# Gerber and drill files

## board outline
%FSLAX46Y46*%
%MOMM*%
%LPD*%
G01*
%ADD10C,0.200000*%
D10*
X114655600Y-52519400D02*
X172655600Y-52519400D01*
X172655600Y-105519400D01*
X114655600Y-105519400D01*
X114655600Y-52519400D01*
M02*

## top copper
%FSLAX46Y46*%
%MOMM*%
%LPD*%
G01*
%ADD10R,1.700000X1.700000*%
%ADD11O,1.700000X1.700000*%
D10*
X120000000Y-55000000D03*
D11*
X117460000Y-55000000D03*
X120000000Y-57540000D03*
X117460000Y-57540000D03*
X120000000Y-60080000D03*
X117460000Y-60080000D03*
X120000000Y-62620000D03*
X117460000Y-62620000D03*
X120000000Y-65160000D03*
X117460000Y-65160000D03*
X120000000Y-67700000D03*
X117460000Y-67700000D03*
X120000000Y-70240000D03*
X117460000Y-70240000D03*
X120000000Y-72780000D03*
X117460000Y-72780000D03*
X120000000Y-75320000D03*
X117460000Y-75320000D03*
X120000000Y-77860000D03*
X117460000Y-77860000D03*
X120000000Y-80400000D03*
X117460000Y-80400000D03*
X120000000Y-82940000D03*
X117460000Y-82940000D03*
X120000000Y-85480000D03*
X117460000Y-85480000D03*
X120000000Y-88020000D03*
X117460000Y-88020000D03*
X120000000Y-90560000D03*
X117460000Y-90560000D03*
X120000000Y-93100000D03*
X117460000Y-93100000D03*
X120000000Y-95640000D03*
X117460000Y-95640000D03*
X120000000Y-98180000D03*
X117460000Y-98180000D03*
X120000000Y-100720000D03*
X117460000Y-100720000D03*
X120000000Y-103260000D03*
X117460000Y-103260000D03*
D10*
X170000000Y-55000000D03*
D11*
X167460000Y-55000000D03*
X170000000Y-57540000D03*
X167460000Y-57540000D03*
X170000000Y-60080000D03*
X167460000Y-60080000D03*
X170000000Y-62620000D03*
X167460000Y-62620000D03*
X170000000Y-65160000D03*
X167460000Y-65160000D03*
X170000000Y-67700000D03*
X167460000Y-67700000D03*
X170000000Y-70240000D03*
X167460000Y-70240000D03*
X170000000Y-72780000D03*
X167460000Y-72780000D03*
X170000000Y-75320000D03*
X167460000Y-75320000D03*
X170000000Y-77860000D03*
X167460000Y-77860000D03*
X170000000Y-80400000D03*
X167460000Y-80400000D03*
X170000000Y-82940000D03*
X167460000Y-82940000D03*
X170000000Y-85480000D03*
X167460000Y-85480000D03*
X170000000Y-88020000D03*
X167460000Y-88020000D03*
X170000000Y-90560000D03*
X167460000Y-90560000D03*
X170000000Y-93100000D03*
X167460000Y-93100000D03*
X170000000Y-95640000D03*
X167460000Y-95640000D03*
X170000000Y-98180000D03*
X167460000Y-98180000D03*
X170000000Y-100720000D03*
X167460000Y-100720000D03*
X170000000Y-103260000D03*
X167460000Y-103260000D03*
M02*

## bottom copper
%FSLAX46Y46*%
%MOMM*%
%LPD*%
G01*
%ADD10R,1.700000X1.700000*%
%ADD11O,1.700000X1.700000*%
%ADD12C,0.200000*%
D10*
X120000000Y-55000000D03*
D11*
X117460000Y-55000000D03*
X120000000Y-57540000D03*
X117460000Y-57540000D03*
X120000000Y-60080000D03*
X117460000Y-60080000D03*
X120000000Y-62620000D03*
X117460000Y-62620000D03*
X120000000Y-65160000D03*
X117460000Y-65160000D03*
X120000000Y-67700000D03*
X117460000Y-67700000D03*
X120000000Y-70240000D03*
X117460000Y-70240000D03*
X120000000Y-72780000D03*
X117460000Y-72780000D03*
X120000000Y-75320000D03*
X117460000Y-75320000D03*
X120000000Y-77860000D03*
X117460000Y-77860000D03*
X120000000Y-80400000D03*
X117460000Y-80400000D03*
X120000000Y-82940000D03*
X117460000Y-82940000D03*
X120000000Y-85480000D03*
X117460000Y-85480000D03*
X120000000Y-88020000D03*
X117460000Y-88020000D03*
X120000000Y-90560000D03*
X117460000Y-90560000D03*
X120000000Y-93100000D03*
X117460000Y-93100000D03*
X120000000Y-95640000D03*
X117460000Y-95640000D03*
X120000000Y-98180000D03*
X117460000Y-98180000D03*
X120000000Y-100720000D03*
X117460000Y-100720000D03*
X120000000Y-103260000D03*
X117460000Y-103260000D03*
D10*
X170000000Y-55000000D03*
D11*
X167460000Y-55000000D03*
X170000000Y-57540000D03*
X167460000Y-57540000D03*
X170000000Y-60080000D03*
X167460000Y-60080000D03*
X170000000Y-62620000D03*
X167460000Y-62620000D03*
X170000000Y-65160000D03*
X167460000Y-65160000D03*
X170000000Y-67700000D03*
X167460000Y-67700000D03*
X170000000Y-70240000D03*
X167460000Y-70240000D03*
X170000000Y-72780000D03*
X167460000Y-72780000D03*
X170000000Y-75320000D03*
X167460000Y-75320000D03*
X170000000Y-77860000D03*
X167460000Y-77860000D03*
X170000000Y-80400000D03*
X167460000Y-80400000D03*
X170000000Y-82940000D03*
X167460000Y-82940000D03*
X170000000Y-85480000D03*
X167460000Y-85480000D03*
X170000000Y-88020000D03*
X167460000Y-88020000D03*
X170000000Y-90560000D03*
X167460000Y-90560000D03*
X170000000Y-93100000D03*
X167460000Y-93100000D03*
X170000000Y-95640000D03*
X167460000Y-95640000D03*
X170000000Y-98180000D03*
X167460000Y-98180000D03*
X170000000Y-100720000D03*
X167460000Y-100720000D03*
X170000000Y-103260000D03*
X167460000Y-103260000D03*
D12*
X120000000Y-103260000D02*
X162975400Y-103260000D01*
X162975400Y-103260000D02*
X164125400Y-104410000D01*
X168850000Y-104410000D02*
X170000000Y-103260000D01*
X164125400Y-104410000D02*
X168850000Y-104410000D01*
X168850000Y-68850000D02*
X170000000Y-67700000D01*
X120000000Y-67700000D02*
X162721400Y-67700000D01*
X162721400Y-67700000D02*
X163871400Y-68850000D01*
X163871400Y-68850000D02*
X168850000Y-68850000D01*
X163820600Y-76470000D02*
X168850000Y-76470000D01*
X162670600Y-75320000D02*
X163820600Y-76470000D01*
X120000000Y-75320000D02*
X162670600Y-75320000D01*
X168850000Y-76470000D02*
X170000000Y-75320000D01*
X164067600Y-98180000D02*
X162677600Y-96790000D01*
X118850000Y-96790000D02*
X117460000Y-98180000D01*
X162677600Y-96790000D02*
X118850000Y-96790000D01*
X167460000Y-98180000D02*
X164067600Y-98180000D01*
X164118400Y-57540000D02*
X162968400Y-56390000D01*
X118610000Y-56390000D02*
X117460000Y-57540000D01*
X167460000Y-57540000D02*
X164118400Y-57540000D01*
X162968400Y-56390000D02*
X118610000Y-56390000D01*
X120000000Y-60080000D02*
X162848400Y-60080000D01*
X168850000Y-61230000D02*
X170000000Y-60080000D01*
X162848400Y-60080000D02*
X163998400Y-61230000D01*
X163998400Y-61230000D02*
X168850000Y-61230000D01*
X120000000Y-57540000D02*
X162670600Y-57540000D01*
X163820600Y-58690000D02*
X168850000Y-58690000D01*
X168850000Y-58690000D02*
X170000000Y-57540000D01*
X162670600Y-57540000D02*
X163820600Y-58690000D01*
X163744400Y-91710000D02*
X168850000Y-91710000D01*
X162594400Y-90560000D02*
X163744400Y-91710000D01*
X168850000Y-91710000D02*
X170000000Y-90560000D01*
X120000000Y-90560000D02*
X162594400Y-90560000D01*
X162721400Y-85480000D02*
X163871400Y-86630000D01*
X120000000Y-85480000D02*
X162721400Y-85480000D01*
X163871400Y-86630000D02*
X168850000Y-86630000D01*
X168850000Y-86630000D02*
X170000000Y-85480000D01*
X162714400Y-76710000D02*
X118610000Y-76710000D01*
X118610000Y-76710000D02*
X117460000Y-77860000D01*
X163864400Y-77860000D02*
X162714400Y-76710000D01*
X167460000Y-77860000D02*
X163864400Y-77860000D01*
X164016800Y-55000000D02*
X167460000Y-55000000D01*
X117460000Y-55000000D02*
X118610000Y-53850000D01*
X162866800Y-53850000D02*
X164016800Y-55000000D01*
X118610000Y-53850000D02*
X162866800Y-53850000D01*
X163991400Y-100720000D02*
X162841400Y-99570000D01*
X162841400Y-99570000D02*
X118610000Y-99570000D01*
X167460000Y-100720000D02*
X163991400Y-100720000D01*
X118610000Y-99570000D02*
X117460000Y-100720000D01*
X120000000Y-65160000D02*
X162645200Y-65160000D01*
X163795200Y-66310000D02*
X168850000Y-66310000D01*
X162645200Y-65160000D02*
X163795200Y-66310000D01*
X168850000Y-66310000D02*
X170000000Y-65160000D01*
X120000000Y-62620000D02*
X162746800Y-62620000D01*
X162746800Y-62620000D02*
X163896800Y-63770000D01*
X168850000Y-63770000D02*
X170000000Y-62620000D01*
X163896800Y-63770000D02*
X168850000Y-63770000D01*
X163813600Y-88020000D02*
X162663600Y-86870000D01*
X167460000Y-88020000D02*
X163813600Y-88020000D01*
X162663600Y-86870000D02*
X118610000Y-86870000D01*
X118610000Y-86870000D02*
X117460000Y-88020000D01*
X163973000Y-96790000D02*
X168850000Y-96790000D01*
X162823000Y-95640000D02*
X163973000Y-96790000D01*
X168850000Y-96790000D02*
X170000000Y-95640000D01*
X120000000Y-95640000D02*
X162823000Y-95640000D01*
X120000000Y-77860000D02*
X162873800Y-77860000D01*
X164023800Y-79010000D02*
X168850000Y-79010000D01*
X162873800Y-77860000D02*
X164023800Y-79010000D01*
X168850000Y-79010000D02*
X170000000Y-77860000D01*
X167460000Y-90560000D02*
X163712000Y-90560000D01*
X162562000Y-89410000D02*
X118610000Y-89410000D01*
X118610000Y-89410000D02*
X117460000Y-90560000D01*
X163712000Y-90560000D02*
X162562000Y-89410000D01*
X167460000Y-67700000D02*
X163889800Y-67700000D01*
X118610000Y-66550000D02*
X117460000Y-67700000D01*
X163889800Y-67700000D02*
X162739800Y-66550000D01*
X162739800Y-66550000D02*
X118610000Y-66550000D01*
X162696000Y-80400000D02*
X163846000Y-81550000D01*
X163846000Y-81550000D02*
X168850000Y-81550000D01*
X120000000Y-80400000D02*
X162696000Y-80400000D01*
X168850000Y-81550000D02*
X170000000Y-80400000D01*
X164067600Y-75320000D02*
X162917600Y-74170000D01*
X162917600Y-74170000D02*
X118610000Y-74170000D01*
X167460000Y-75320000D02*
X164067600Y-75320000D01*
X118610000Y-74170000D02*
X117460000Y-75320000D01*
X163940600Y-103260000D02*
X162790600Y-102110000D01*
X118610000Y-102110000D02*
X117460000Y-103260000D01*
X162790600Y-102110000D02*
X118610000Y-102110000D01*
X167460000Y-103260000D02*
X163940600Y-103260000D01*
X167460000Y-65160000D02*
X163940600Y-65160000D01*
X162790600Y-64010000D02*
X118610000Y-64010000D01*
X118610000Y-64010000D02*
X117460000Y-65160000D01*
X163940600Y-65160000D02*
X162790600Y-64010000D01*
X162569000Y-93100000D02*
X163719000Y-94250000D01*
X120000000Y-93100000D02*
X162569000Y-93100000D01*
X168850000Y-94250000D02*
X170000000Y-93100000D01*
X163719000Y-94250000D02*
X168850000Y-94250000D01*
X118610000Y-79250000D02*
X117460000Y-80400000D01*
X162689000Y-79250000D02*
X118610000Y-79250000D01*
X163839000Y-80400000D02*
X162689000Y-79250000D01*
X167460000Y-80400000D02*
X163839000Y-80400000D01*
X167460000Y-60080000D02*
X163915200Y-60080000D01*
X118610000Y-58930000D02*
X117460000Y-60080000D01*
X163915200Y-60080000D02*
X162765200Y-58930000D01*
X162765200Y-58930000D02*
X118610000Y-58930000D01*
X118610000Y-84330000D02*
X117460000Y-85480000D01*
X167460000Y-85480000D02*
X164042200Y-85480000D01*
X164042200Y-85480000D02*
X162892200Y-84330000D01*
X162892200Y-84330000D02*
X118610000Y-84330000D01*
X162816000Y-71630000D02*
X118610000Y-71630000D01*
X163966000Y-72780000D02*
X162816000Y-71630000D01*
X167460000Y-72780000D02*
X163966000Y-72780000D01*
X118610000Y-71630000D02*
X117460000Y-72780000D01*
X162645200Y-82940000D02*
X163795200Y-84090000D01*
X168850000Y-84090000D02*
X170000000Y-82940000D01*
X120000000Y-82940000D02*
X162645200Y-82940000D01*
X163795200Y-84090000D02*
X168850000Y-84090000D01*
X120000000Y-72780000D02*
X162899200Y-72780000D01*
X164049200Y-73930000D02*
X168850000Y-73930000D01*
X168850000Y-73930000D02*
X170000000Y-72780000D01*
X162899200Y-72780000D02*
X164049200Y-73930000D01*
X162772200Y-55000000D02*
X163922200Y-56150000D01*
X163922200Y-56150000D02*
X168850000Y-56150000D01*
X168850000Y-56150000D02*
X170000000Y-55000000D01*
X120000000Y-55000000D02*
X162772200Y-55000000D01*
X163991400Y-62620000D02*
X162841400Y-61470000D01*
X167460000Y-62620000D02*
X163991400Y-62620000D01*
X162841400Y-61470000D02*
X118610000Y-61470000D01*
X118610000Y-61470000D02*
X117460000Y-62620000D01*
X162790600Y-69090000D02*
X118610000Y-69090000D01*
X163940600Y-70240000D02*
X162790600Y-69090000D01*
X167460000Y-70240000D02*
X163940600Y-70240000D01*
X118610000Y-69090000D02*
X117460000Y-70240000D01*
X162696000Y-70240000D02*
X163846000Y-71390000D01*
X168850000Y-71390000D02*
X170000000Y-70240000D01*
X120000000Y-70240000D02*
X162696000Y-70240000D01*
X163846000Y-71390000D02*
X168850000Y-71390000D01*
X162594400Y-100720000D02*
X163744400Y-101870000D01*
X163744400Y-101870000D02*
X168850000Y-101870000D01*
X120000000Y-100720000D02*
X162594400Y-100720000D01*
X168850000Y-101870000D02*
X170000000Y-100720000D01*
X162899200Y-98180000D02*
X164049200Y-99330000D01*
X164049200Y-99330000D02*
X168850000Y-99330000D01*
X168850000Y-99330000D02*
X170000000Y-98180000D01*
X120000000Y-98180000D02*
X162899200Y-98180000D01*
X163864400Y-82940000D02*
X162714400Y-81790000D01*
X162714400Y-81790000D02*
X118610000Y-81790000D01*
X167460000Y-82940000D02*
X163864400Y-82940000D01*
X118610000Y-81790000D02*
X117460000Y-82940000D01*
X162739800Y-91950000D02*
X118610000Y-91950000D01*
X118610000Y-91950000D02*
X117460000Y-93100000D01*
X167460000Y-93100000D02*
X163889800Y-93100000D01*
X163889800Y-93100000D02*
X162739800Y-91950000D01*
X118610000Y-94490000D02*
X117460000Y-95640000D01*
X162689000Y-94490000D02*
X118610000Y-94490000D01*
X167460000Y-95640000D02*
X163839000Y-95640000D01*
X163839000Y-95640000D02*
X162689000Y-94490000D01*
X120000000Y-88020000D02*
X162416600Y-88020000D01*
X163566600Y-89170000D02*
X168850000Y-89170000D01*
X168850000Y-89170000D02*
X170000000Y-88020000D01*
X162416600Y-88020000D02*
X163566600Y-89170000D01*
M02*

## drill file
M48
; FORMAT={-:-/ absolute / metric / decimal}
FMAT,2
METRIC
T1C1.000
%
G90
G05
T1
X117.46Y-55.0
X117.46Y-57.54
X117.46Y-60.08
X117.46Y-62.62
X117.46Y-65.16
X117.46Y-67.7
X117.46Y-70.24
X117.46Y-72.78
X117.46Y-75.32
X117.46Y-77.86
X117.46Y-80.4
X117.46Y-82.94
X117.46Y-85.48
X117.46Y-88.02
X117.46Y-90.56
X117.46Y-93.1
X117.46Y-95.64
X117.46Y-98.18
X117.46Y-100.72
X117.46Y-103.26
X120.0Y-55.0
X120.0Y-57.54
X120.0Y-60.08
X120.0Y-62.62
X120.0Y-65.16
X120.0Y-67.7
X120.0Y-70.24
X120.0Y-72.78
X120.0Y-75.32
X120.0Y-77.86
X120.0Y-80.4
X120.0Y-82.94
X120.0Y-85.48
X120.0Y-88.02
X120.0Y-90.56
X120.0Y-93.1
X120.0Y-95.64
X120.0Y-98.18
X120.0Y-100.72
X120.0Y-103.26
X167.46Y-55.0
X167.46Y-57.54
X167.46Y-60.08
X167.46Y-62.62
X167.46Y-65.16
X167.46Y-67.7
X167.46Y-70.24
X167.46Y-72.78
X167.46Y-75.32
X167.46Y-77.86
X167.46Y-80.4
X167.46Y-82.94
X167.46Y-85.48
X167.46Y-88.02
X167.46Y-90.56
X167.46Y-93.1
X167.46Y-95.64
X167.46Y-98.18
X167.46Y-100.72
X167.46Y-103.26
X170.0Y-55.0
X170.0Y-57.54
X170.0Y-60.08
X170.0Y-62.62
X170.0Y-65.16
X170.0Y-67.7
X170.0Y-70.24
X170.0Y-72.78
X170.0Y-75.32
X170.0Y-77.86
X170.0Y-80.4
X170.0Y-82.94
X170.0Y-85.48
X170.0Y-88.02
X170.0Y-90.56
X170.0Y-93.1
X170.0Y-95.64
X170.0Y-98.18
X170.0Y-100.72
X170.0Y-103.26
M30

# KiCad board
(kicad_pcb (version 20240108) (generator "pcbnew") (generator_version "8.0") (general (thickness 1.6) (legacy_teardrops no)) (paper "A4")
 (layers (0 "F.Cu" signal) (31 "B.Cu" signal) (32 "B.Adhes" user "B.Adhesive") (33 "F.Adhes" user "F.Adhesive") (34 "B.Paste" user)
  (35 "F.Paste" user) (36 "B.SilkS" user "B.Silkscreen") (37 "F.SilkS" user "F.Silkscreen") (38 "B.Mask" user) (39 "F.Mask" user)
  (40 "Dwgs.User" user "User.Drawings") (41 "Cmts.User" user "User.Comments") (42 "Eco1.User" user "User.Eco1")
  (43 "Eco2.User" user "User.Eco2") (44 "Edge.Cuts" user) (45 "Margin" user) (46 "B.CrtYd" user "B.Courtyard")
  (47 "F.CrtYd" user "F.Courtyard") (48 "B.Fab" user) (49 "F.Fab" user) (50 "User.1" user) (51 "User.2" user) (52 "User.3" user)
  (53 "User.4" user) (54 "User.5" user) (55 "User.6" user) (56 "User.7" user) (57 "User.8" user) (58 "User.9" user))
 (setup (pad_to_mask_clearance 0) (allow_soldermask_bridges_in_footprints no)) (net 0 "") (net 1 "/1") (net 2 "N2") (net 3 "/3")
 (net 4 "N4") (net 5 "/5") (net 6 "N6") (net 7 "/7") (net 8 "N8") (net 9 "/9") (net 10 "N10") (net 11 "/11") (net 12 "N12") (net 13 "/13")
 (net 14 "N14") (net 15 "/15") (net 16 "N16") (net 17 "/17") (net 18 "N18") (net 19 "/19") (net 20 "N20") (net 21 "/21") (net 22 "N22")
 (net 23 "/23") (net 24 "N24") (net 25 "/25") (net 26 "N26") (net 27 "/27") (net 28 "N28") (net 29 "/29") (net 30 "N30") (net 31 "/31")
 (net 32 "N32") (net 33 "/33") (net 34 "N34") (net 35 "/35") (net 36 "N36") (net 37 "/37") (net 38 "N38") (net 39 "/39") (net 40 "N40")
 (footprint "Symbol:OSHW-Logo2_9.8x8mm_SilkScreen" (layer "F.Cu") (at 160.274 97.8408 90)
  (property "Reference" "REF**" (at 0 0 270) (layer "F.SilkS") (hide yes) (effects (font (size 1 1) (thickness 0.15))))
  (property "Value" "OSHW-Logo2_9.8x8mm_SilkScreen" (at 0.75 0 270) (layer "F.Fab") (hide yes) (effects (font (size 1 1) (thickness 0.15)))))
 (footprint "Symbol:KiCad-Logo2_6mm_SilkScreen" (layer "F.Cu") (at 159.512 62.7634 90)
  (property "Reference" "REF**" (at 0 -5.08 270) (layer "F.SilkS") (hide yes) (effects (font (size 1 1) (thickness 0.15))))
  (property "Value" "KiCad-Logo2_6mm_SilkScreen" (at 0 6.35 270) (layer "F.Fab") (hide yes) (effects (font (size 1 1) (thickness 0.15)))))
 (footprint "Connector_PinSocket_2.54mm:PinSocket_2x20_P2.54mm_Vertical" (layer "F.Cu") (at 120 55)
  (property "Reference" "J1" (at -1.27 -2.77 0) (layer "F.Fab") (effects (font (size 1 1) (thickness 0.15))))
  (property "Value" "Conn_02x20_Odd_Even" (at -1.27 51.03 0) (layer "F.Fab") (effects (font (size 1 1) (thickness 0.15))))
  (pad "1" thru_hole rect (at 0 0) (size 1.7 1.7) (drill 1) (layers "*.Cu" "*.Mask") (remove_unused_layers no) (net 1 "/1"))
  (pad "2" thru_hole oval (at -2.54 0) (size 1.7 1.7) (drill 1) (layers "*.Cu" "*.Mask") (remove_unused_layers no) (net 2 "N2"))
  (pad "3" thru_hole oval (at 0 2.54) (size 1.7 1.7) (drill 1) (layers "*.Cu" "*.Mask") (remove_unused_layers no) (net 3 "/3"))
  (pad "4" thru_hole oval (at -2.54 2.54) (size 1.7 1.7) (drill 1) (layers "*.Cu" "*.Mask") (remove_unused_layers no) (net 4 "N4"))
  (pad "5" thru_hole oval (at 0 5.08) (size 1.7 1.7) (drill 1) (layers "*.Cu" "*.Mask") (remove_unused_layers no) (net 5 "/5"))
  (pad "6" thru_hole oval (at -2.54 5.08) (size 1.7 1.7) (drill 1) (layers "*.Cu" "*.Mask") (remove_unused_layers no) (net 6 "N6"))
  (pad "7" thru_hole oval (at 0 7.62) (size 1.7 1.7) (drill 1) (layers "*.Cu" "*.Mask") (remove_unused_layers no) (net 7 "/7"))
  (pad "8" thru_hole oval (at -2.54 7.62) (size 1.7 1.7) (drill 1) (layers "*.Cu" "*.Mask") (remove_unused_layers no) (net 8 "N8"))
  (pad "9" thru_hole oval (at 0 10.16) (size 1.7 1.7) (drill 1) (layers "*.Cu" "*.Mask") (remove_unused_layers no) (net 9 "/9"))
  (pad "10" thru_hole oval (at -2.54 10.16) (size 1.7 1.7) (drill 1) (layers "*.Cu" "*.Mask") (remove_unused_layers no) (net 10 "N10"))
  (pad "11" thru_hole oval (at 0 12.7) (size 1.7 1.7) (drill 1) (layers "*.Cu" "*.Mask") (remove_unused_layers no) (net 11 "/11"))
  (pad "12" thru_hole oval (at -2.54 12.7) (size 1.7 1.7) (drill 1) (layers "*.Cu" "*.Mask") (remove_unused_layers no) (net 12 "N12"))
  (pad "13" thru_hole oval (at 0 15.24) (size 1.7 1.7) (drill 1) (layers "*.Cu" "*.Mask") (remove_unused_layers no) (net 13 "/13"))
  (pad "14" thru_hole oval (at -2.54 15.24) (size 1.7 1.7) (drill 1) (layers "*.Cu" "*.Mask") (remove_unused_layers no) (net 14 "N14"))
  (pad "15" thru_hole oval (at 0 17.78) (size 1.7 1.7) (drill 1) (layers "*.Cu" "*.Mask") (remove_unused_layers no) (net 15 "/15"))
  (pad "16" thru_hole oval (at -2.54 17.78) (size 1.7 1.7) (drill 1) (layers "*.Cu" "*.Mask") (remove_unused_layers no) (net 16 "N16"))
  (pad "17" thru_hole oval (at 0 20.32) (size 1.7 1.7) (drill 1) (layers "*.Cu" "*.Mask") (remove_unused_layers no) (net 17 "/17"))
  (pad "18" thru_hole oval (at -2.54 20.32) (size 1.7 1.7) (drill 1) (layers "*.Cu" "*.Mask") (remove_unused_layers no) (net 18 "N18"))
  (pad "19" thru_hole oval (at 0 22.86) (size 1.7 1.7) (drill 1) (layers "*.Cu" "*.Mask") (remove_unused_layers no) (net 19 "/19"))
  (pad "20" thru_hole oval (at -2.54 22.86) (size 1.7 1.7) (drill 1) (layers "*.Cu" "*.Mask") (remove_unused_layers no) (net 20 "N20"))
  (pad "21" thru_hole oval (at 0 25.4) (size 1.7 1.7) (drill 1) (layers "*.Cu" "*.Mask") (remove_unused_layers no) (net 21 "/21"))
  (pad "22" thru_hole oval (at -2.54 25.4) (size 1.7 1.7) (drill 1) (layers "*.Cu" "*.Mask") (remove_unused_layers no) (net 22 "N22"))
  (pad "23" thru_hole oval (at 0 27.94) (size 1.7 1.7) (drill 1) (layers "*.Cu" "*.Mask") (remove_unused_layers no) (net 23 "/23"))
  (pad "24" thru_hole oval (at -2.54 27.94) (size 1.7 1.7) (drill 1) (layers "*.Cu" "*.Mask") (remove_unused_layers no) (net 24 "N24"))
  (pad "25" thru_hole oval (at 0 30.48) (size 1.7 1.7) (drill 1) (layers "*.Cu" "*.Mask") (remove_unused_layers no) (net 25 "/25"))
  (pad "26" thru_hole oval (at -2.54 30.48) (size 1.7 1.7) (drill 1) (layers "*.Cu" "*.Mask") (remove_unused_layers no) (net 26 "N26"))
  (pad "27" thru_hole oval (at 0 33.02) (size 1.7 1.7) (drill 1) (layers "*.Cu" "*.Mask") (remove_unused_layers no) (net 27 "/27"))
  (pad "28" thru_hole oval (at -2.54 33.02) (size 1.7 1.7) (drill 1) (layers "*.Cu" "*.Mask") (remove_unused_layers no) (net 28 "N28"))
  (pad "29" thru_hole oval (at 0 35.56) (size 1.7 1.7) (drill 1) (layers "*.Cu" "*.Mask") (remove_unused_layers no) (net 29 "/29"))
  (pad "30" thru_hole oval (at -2.54 35.56) (size 1.7 1.7) (drill 1) (layers "*.Cu" "*.Mask") (remove_unused_layers no) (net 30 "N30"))
  (pad "31" thru_hole oval (at 0 38.1) (size 1.7 1.7) (drill 1) (layers "*.Cu" "*.Mask") (remove_unused_layers no) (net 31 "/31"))
  (pad "32" thru_hole oval (at -2.54 38.1) (size 1.7 1.7) (drill 1) (layers "*.Cu" "*.Mask") (remove_unused_layers no) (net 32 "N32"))
  (pad "33" thru_hole oval (at 0 40.64) (size 1.7 1.7) (drill 1) (layers "*.Cu" "*.Mask") (remove_unused_layers no) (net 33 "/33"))
  (pad "34" thru_hole oval (at -2.54 40.64) (size 1.7 1.7) (drill 1) (layers "*.Cu" "*.Mask") (remove_unused_layers no) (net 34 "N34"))
  (pad "35" thru_hole oval (at 0 43.18) (size 1.7 1.7) (drill 1) (layers "*.Cu" "*.Mask") (remove_unused_layers no) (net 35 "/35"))
  (pad "36" thru_hole oval (at -2.54 43.18) (size 1.7 1.7) (drill 1) (layers "*.Cu" "*.Mask") (remove_unused_layers no) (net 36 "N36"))
  (pad "37" thru_hole oval (at 0 45.72) (size 1.7 1.7) (drill 1) (layers "*.Cu" "*.Mask") (remove_unused_layers no) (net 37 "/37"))
  (pad "38" thru_hole oval (at -2.54 45.72) (size 1.7 1.7) (drill 1) (layers "*.Cu" "*.Mask") (remove_unused_layers no) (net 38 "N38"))
  (pad "39" thru_hole oval (at 0 48.26) (size 1.7 1.7) (drill 1) (layers "*.Cu" "*.Mask") (remove_unused_layers no) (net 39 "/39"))
  (pad "40" thru_hole oval (at -2.54 48.26) (size 1.7 1.7) (drill 1) (layers "*.Cu" "*.Mask") (remove_unused_layers no) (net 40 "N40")))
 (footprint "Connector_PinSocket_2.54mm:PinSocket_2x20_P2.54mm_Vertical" (layer "F.Cu") (at 170 55)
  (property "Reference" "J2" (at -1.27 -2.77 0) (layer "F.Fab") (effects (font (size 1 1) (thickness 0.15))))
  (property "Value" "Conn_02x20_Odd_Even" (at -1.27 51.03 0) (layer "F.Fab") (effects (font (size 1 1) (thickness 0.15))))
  (pad "1" thru_hole rect (at 0 0) (size 1.7 1.7) (drill 1) (layers "*.Cu" "*.Mask") (remove_unused_layers no) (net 1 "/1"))
  (pad "2" thru_hole oval (at -2.54 0) (size 1.7 1.7) (drill 1) (layers "*.Cu" "*.Mask") (remove_unused_layers no) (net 2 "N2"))
  (pad "3" thru_hole oval (at 0 2.54) (size 1.7 1.7) (drill 1) (layers "*.Cu" "*.Mask") (remove_unused_layers no) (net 3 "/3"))
  (pad "4" thru_hole oval (at -2.54 2.54) (size 1.7 1.7) (drill 1) (layers "*.Cu" "*.Mask") (remove_unused_layers no) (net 4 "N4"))
  (pad "5" thru_hole oval (at 0 5.08) (size 1.7 1.7) (drill 1) (layers "*.Cu" "*.Mask") (remove_unused_layers no) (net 5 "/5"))
  (pad "6" thru_hole oval (at -2.54 5.08) (size 1.7 1.7) (drill 1) (layers "*.Cu" "*.Mask") (remove_unused_layers no) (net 6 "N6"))
  (pad "7" thru_hole oval (at 0 7.62) (size 1.7 1.7) (drill 1) (layers "*.Cu" "*.Mask") (remove_unused_layers no) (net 7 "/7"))
  (pad "8" thru_hole oval (at -2.54 7.62) (size 1.7 1.7) (drill 1) (layers "*.Cu" "*.Mask") (remove_unused_layers no) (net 8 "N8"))
  (pad "9" thru_hole oval (at 0 10.16) (size 1.7 1.7) (drill 1) (layers "*.Cu" "*.Mask") (remove_unused_layers no) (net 9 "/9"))
  (pad "10" thru_hole oval (at -2.54 10.16) (size 1.7 1.7) (drill 1) (layers "*.Cu" "*.Mask") (remove_unused_layers no) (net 10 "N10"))
  (pad "11" thru_hole oval (at 0 12.7) (size 1.7 1.7) (drill 1) (layers "*.Cu" "*.Mask") (remove_unused_layers no) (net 11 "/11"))
  (pad "12" thru_hole oval (at -2.54 12.7) (size 1.7 1.7) (drill 1) (layers "*.Cu" "*.Mask") (remove_unused_layers no) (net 12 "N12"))
  (pad "13" thru_hole oval (at 0 15.24) (size 1.7 1.7) (drill 1) (layers "*.Cu" "*.Mask") (remove_unused_layers no) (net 13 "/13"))
  (pad "14" thru_hole oval (at -2.54 15.24) (size 1.7 1.7) (drill 1) (layers "*.Cu" "*.Mask") (remove_unused_layers no) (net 14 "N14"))
  (pad "15" thru_hole oval (at 0 17.78) (size 1.7 1.7) (drill 1) (layers "*.Cu" "*.Mask") (remove_unused_layers no) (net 15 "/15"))
  (pad "16" thru_hole oval (at -2.54 17.78) (size 1.7 1.7) (drill 1) (layers "*.Cu" "*.Mask") (remove_unused_layers no) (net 16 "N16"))
  (pad "17" thru_hole oval (at 0 20.32) (size 1.7 1.7) (drill 1) (layers "*.Cu" "*.Mask") (remove_unused_layers no) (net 17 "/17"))
  (pad "18" thru_hole oval (at -2.54 20.32) (size 1.7 1.7) (drill 1) (layers "*.Cu" "*.Mask") (remove_unused_layers no) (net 18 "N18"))
  (pad "19" thru_hole oval (at 0 22.86) (size 1.7 1.7) (drill 1) (layers "*.Cu" "*.Mask") (remove_unused_layers no) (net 19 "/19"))
  (pad "20" thru_hole oval (at -2.54 22.86) (size 1.7 1.7) (drill 1) (layers "*.Cu" "*.Mask") (remove_unused_layers no) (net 20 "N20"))
  (pad "21" thru_hole oval (at 0 25.4) (size 1.7 1.7) (drill 1) (layers "*.Cu" "*.Mask") (remove_unused_layers no) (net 21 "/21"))
  (pad "22" thru_hole oval (at -2.54 25.4) (size 1.7 1.7) (drill 1) (layers "*.Cu" "*.Mask") (remove_unused_layers no) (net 22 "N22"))
  (pad "23" thru_hole oval (at 0 27.94) (size 1.7 1.7) (drill 1) (layers "*.Cu" "*.Mask") (remove_unused_layers no) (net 23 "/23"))
  (pad "24" thru_hole oval (at -2.54 27.94) (size 1.7 1.7) (drill 1) (layers "*.Cu" "*.Mask") (remove_unused_layers no) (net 24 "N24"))
  (pad "25" thru_hole oval (at 0 30.48) (size 1.7 1.7) (drill 1) (layers "*.Cu" "*.Mask") (remove_unused_layers no) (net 25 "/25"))
  (pad "26" thru_hole oval (at -2.54 30.48) (size 1.7 1.7) (drill 1) (layers "*.Cu" "*.Mask") (remove_unused_layers no) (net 26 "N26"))
  (pad "27" thru_hole oval (at 0 33.02) (size 1.7 1.7) (drill 1) (layers "*.Cu" "*.Mask") (remove_unused_layers no) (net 27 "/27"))
  (pad "28" thru_hole oval (at -2.54 33.02) (size 1.7 1.7) (drill 1) (layers "*.Cu" "*.Mask") (remove_unused_layers no) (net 28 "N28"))
  (pad "29" thru_hole oval (at 0 35.56) (size 1.7 1.7) (drill 1) (layers "*.Cu" "*.Mask") (remove_unused_layers no) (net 29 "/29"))
  (pad "30" thru_hole oval (at -2.54 35.56) (size 1.7 1.7) (drill 1) (layers "*.Cu" "*.Mask") (remove_unused_layers no) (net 30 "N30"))
  (pad "31" thru_hole oval (at 0 38.1) (size 1.7 1.7) (drill 1) (layers "*.Cu" "*.Mask") (remove_unused_layers no) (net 31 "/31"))
  (pad "32" thru_hole oval (at -2.54 38.1) (size 1.7 1.7) (drill 1) (layers "*.Cu" "*.Mask") (remove_unused_layers no) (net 32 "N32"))
  (pad "33" thru_hole oval (at 0 40.64) (size 1.7 1.7) (drill 1) (layers "*.Cu" "*.Mask") (remove_unused_layers no) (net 33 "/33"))
  (pad "34" thru_hole oval (at -2.54 40.64) (size 1.7 1.7) (drill 1) (layers "*.Cu" "*.Mask") (remove_unused_layers no) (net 34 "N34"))
  (pad "35" thru_hole oval (at 0 43.18) (size 1.7 1.7) (drill 1) (layers "*.Cu" "*.Mask") (remove_unused_layers no) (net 35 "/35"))
  (pad "36" thru_hole oval (at -2.54 43.18) (size 1.7 1.7) (drill 1) (layers "*.Cu" "*.Mask") (remove_unused_layers no) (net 36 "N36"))
  (pad "37" thru_hole oval (at 0 45.72) (size 1.7 1.7) (drill 1) (layers "*.Cu" "*.Mask") (remove_unused_layers no) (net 37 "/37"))
  (pad "38" thru_hole oval (at -2.54 45.72) (size 1.7 1.7) (drill 1) (layers "*.Cu" "*.Mask") (remove_unused_layers no) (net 38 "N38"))
  (pad "39" thru_hole oval (at 0 48.26) (size 1.7 1.7) (drill 1) (layers "*.Cu" "*.Mask") (remove_unused_layers no) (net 39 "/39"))
  (pad "40" thru_hole oval (at -2.54 48.26) (size 1.7 1.7) (drill 1) (layers "*.Cu" "*.Mask") (remove_unused_layers no) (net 40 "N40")))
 (gr_rect (start 114.6556 52.5194) (end 172.6556 105.5194) (stroke (width 0.2) (type default)) (fill none) (layer "Edge.Cuts"))
 (segment (start 120 103.26) (end 162.9754 103.26) (width 0.2) (layer "B.Cu") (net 39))
 (segment (start 162.9754 103.26) (end 164.1254 104.41) (width 0.2) (layer "B.Cu") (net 39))
 (segment (start 168.85 104.41) (end 170 103.26) (width 0.2) (layer "B.Cu") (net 39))
 (segment (start 164.1254 104.41) (end 168.85 104.41) (width 0.2) (layer "B.Cu") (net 39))
 (segment (start 168.85 68.85) (end 170 67.7) (width 0.2) (layer "B.Cu") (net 11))
 (segment (start 120 67.7) (end 162.7214 67.7) (width 0.2) (layer "B.Cu") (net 11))
 (segment (start 162.7214 67.7) (end 163.8714 68.85) (width 0.2) (layer "B.Cu") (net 11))
 (segment (start 163.8714 68.85) (end 168.85 68.85) (width 0.2) (layer "B.Cu") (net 11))
 (segment (start 163.8206 76.47) (end 168.85 76.47) (width 0.2) (layer "B.Cu") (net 17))
 (segment (start 162.6706 75.32) (end 163.8206 76.47) (width 0.2) (layer "B.Cu") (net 17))
 (segment (start 120 75.32) (end 162.6706 75.32) (width 0.2) (layer "B.Cu") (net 17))
 (segment (start 168.85 76.47) (end 170 75.32) (width 0.2) (layer "B.Cu") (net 17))
 (segment (start 164.0676 98.18) (end 162.6776 96.79) (width 0.2) (layer "B.Cu") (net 36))
 (segment (start 118.85 96.79) (end 117.46 98.18) (width 0.2) (layer "B.Cu") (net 36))
 (segment (start 162.6776 96.79) (end 118.85 96.79) (width 0.2) (layer "B.Cu") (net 36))
 (segment (start 167.46 98.18) (end 164.0676 98.18) (width 0.2) (layer "B.Cu") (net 36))
 (segment (start 164.1184 57.54) (end 162.9684 56.39) (width 0.2) (layer "B.Cu") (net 4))
 (segment (start 118.61 56.39) (end 117.46 57.54) (width 0.2) (layer "B.Cu") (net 4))
 (segment (start 167.46 57.54) (end 164.1184 57.54) (width 0.2) (layer "B.Cu") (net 4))
 (segment (start 162.9684 56.39) (end 118.61 56.39) (width 0.2) (layer "B.Cu") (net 4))
 (segment (start 120 60.08) (end 162.8484 60.08) (width 0.2) (layer "B.Cu") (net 5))
 (segment (start 168.85 61.23) (end 170 60.08) (width 0.2) (layer "B.Cu") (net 5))
 (segment (start 162.8484 60.08) (end 163.9984 61.23) (width 0.2) (layer "B.Cu") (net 5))
 (segment (start 163.9984 61.23) (end 168.85 61.23) (width 0.2) (layer "B.Cu") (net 5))
 (segment (start 120 57.54) (end 162.6706 57.54) (width 0.2) (layer "B.Cu") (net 3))
 (segment (start 163.8206 58.69) (end 168.85 58.69) (width 0.2) (layer "B.Cu") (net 3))
 (segment (start 168.85 58.69) (end 170 57.54) (width 0.2) (layer "B.Cu") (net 3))
 (segment (start 162.6706 57.54) (end 163.8206 58.69) (width 0.2) (layer "B.Cu") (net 3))
 (segment (start 163.7444 91.71) (end 168.85 91.71) (width 0.2) (layer "B.Cu") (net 29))
 (segment (start 162.5944 90.56) (end 163.7444 91.71) (width 0.2) (layer "B.Cu") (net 29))
 (segment (start 168.85 91.71) (end 170 90.56) (width 0.2) (layer "B.Cu") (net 29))
 (segment (start 120 90.56) (end 162.5944 90.56) (width 0.2) (layer "B.Cu") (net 29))
 (segment (start 162.7214 85.48) (end 163.8714 86.63) (width 0.2) (layer "B.Cu") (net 25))
 (segment (start 120 85.48) (end 162.7214 85.48) (width 0.2) (layer "B.Cu") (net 25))
 (segment (start 163.8714 86.63) (end 168.85 86.63) (width 0.2) (layer "B.Cu") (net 25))
 (segment (start 168.85 86.63) (end 170 85.48) (width 0.2) (layer "B.Cu") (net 25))
 (segment (start 162.7144 76.71) (end 118.61 76.71) (width 0.2) (layer "B.Cu") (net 20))
 (segment (start 118.61 76.71) (end 117.46 77.86) (width 0.2) (layer "B.Cu") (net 20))
 (segment (start 163.8644 77.86) (end 162.7144 76.71) (width 0.2) (layer "B.Cu") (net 20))
 (segment (start 167.46 77.86) (end 163.8644 77.86) (width 0.2) (layer "B.Cu") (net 20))
 (segment (start 164.0168 55) (end 167.46 55) (width 0.2) (layer "B.Cu") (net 2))
 (segment (start 117.46 55) (end 118.61 53.85) (width 0.2) (layer "B.Cu") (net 2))
 (segment (start 162.8668 53.85) (end 164.0168 55) (width 0.2) (layer "B.Cu") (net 2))
 (segment (start 118.61 53.85) (end 162.8668 53.85) (width 0.2) (layer "B.Cu") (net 2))
 (segment (start 163.9914 100.72) (end 162.8414 99.57) (width 0.2) (layer "B.Cu") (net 38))
 (segment (start 162.8414 99.57) (end 118.61 99.57) (width 0.2) (layer "B.Cu") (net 38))
 (segment (start 167.46 100.72) (end 163.9914 100.72) (width 0.2) (layer "B.Cu") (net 38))
 (segment (start 118.61 99.57) (end 117.46 100.72) (width 0.2) (layer "B.Cu") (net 38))
 (segment (start 120 65.16) (end 162.6452 65.16) (width 0.2) (layer "B.Cu") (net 9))
 (segment (start 163.7952 66.31) (end 168.85 66.31) (width 0.2) (layer "B.Cu") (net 9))
 (segment (start 162.6452 65.16) (end 163.7952 66.31) (width 0.2) (layer "B.Cu") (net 9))
 (segment (start 168.85 66.31) (end 170 65.16) (width 0.2) (layer "B.Cu") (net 9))
 (segment (start 120 62.62) (end 162.7468 62.62) (width 0.2) (layer "B.Cu") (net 7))
 (segment (start 162.7468 62.62) (end 163.8968 63.77) (width 0.2) (layer "B.Cu") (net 7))
 (segment (start 168.85 63.77) (end 170 62.62) (width 0.2) (layer "B.Cu") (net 7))
 (segment (start 163.8968 63.77) (end 168.85 63.77) (width 0.2) (layer "B.Cu") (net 7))
 (segment (start 163.8136 88.02) (end 162.6636 86.87) (width 0.2) (layer "B.Cu") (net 28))
 (segment (start 167.46 88.02) (end 163.8136 88.02) (width 0.2) (layer "B.Cu") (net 28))
 (segment (start 162.6636 86.87) (end 118.61 86.87) (width 0.2) (layer "B.Cu") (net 28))
 (segment (start 118.61 86.87) (end 117.46 88.02) (width 0.2) (layer "B.Cu") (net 28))
 (segment (start 163.973 96.79) (end 168.85 96.79) (width 0.2) (layer "B.Cu") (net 33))
 (segment (start 162.823 95.64) (end 163.973 96.79) (width 0.2) (layer "B.Cu") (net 33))
 (segment (start 168.85 96.79) (end 170 95.64) (width 0.2) (layer "B.Cu") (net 33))
 (segment (start 120 95.64) (end 162.823 95.64) (width 0.2) (layer "B.Cu") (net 33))
 (segment (start 120 77.86) (end 162.8738 77.86) (width 0.2) (layer "B.Cu") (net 19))
 (segment (start 164.0238 79.01) (end 168.85 79.01) (width 0.2) (layer "B.Cu") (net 19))
 (segment (start 162.8738 77.86) (end 164.0238 79.01) (width 0.2) (layer "B.Cu") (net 19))
 (segment (start 168.85 79.01) (end 170 77.86) (width 0.2) (layer "B.Cu") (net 19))
 (segment (start 167.46 90.56) (end 163.712 90.56) (width 0.2) (layer "B.Cu") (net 30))
 (segment (start 162.562 89.41) (end 118.61 89.41) (width 0.2) (layer "B.Cu") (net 30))
 (segment (start 118.61 89.41) (end 117.46 90.56) (width 0.2) (layer "B.Cu") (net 30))
 (segment (start 163.712 90.56) (end 162.562 89.41) (width 0.2) (layer "B.Cu") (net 30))
 (segment (start 167.46 67.7) (end 163.8898 67.7) (width 0.2) (layer "B.Cu") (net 12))
 (segment (start 118.61 66.55) (end 117.46 67.7) (width 0.2) (layer "B.Cu") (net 12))
 (segment (start 163.8898 67.7) (end 162.7398 66.55) (width 0.2) (layer "B.Cu") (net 12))
 (segment (start 162.7398 66.55) (end 118.61 66.55) (width 0.2) (layer "B.Cu") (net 12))
 (segment (start 162.696 80.4) (end 163.846 81.55) (width 0.2) (layer "B.Cu") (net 21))
 (segment (start 163.846 81.55) (end 168.85 81.55) (width 0.2) (layer "B.Cu") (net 21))
 (segment (start 120 80.4) (end 162.696 80.4) (width 0.2) (layer "B.Cu") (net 21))
 (segment (start 168.85 81.55) (end 170 80.4) (width 0.2) (layer "B.Cu") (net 21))
 (segment (start 164.0676 75.32) (end 162.9176 74.17) (width 0.2) (layer "B.Cu") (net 18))
 (segment (start 162.9176 74.17) (end 118.61 74.17) (width 0.2) (layer "B.Cu") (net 18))
 (segment (start 167.46 75.32) (end 164.0676 75.32) (width 0.2) (layer "B.Cu") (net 18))
 (segment (start 118.61 74.17) (end 117.46 75.32) (width 0.2) (layer "B.Cu") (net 18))
 (segment (start 163.9406 103.26) (end 162.7906 102.11) (width 0.2) (layer "B.Cu") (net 40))
 (segment (start 118.61 102.11) (end 117.46 103.26) (width 0.2) (layer "B.Cu") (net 40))
 (segment (start 162.7906 102.11) (end 118.61 102.11) (width 0.2) (layer "B.Cu") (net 40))
 (segment (start 167.46 103.26) (end 163.9406 103.26) (width 0.2) (layer "B.Cu") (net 40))
 (segment (start 167.46 65.16) (end 163.9406 65.16) (width 0.2) (layer "B.Cu") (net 10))
 (segment (start 162.7906 64.01) (end 118.61 64.01) (width 0.2) (layer "B.Cu") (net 10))
 (segment (start 118.61 64.01) (end 117.46 65.16) (width 0.2) (layer "B.Cu") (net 10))
 (segment (start 163.9406 65.16) (end 162.7906 64.01) (width 0.2) (layer "B.Cu") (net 10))
 (segment (start 162.569 93.1) (end 163.719 94.25) (width 0.2) (layer "B.Cu") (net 31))
 (segment (start 120 93.1) (end 162.569 93.1) (width 0.2) (layer "B.Cu") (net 31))
 (segment (start 168.85 94.25) (end 170 93.1) (width 0.2) (layer "B.Cu") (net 31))
 (segment (start 163.719 94.25) (end 168.85 94.25) (width 0.2) (layer "B.Cu") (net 31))
 (segment (start 118.61 79.25) (end 117.46 80.4) (width 0.2) (layer "B.Cu") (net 22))
 (segment (start 162.689 79.25) (end 118.61 79.25) (width 0.2) (layer "B.Cu") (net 22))
 (segment (start 163.839 80.4) (end 162.689 79.25) (width 0.2) (layer "B.Cu") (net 22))
 (segment (start 167.46 80.4) (end 163.839 80.4) (width 0.2) (layer "B.Cu") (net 22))
 (segment (start 167.46 60.08) (end 163.9152 60.08) (width 0.2) (layer "B.Cu") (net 6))
 (segment (start 118.61 58.93) (end 117.46 60.08) (width 0.2) (layer "B.Cu") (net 6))
 (segment (start 163.9152 60.08) (end 162.7652 58.93) (width 0.2) (layer "B.Cu") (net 6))
 (segment (start 162.7652 58.93) (end 118.61 58.93) (width 0.2) (layer "B.Cu") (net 6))
 (segment (start 118.61 84.33) (end 117.46 85.48) (width 0.2) (layer "B.Cu") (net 26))
 (segment (start 167.46 85.48) (end 164.0422 85.48) (width 0.2) (layer "B.Cu") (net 26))
 (segment (start 164.0422 85.48) (end 162.8922 84.33) (width 0.2) (layer "B.Cu") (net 26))
 (segment (start 162.8922 84.33) (end 118.61 84.33) (width 0.2) (layer "B.Cu") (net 26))
 (segment (start 162.816 71.63) (end 118.61 71.63) (width 0.2) (layer "B.Cu") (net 16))
 (segment (start 163.966 72.78) (end 162.816 71.63) (width 0.2) (layer "B.Cu") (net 16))
 (segment (start 167.46 72.78) (end 163.966 72.78) (width 0.2) (layer "B.Cu") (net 16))
 (segment (start 118.61 71.63) (end 117.46 72.78) (width 0.2) (layer "B.Cu") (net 16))
 (segment (start 162.6452 82.94) (end 163.7952 84.09) (width 0.2) (layer "B.Cu") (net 23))
 (segment (start 168.85 84.09) (end 170 82.94) (width 0.2) (layer "B.Cu") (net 23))
 (segment (start 120 82.94) (end 162.6452 82.94) (width 0.2) (layer "B.Cu") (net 23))
 (segment (start 163.7952 84.09) (end 168.85 84.09) (width 0.2) (layer "B.Cu") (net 23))
 (segment (start 120 72.78) (end 162.8992 72.78) (width 0.2) (layer "B.Cu") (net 15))
 (segment (start 164.0492 73.93) (end 168.85 73.93) (width 0.2) (layer "B.Cu") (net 15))
 (segment (start 168.85 73.93) (end 170 72.78) (width 0.2) (layer "B.Cu") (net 15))
 (segment (start 162.8992 72.78) (end 164.0492 73.93) (width 0.2) (layer "B.Cu") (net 15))
 (segment (start 162.7722 55) (end 163.9222 56.15) (width 0.2) (layer "B.Cu") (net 1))
 (segment (start 163.9222 56.15) (end 168.85 56.15) (width 0.2) (layer "B.Cu") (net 1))
 (segment (start 168.85 56.15) (end 170 55) (width 0.2) (layer "B.Cu") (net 1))
 (segment (start 120 55) (end 162.7722 55) (width 0.2) (layer "B.Cu") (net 1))
 (segment (start 163.9914 62.62) (end 162.8414 61.47) (width 0.2) (layer "B.Cu") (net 8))
 (segment (start 167.46 62.62) (end 163.9914 62.62) (width 0.2) (layer "B.Cu") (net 8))
 (segment (start 162.8414 61.47) (end 118.61 61.47) (width 0.2) (layer "B.Cu") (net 8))
 (segment (start 118.61 61.47) (end 117.46 62.62) (width 0.2) (layer "B.Cu") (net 8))
 (segment (start 162.7906 69.09) (end 118.61 69.09) (width 0.2) (layer "B.Cu") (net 14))
 (segment (start 163.9406 70.24) (end 162.7906 69.09) (width 0.2) (layer "B.Cu") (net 14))
 (segment (start 167.46 70.24) (end 163.9406 70.24) (width 0.2) (layer "B.Cu") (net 14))
 (segment (start 118.61 69.09) (end 117.46 70.24) (width 0.2) (layer "B.Cu") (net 14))
 (segment (start 162.696 70.24) (end 163.846 71.39) (width 0.2) (layer "B.Cu") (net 13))
 (segment (start 168.85 71.39) (end 170 70.24) (width 0.2) (layer "B.Cu") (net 13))
 (segment (start 120 70.24) (end 162.696 70.24) (width 0.2) (layer "B.Cu") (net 13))
 (segment (start 163.846 71.39) (end 168.85 71.39) (width 0.2) (layer "B.Cu") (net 13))
 (segment (start 162.5944 100.72) (end 163.7444 101.87) (width 0.2) (layer "B.Cu") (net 37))
 (segment (start 163.7444 101.87) (end 168.85 101.87) (width 0.2) (layer "B.Cu") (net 37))
 (segment (start 120 100.72) (end 162.5944 100.72) (width 0.2) (layer "B.Cu") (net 37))
 (segment (start 168.85 101.87) (end 170 100.72) (width 0.2) (layer "B.Cu") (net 37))
 (segment (start 162.8992 98.18) (end 164.0492 99.33) (width 0.2) (layer "B.Cu") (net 35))
 (segment (start 164.0492 99.33) (end 168.85 99.33) (width 0.2) (layer "B.Cu") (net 35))
 (segment (start 168.85 99.33) (end 170 98.18) (width 0.2) (layer "B.Cu") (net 35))
 (segment (start 120 98.18) (end 162.8992 98.18) (width 0.2) (layer "B.Cu") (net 35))
 (segment (start 163.8644 82.94) (end 162.7144 81.79) (width 0.2) (layer "B.Cu") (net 24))
 (segment (start 162.7144 81.79) (end 118.61 81.79) (width 0.2) (layer "B.Cu") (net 24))
 (segment (start 167.46 82.94) (end 163.8644 82.94) (width 0.2) (layer "B.Cu") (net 24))
 (segment (start 118.61 81.79) (end 117.46 82.94) (width 0.2) (layer "B.Cu") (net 24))
 (segment (start 162.7398 91.95) (end 118.61 91.95) (width 0.2) (layer "B.Cu") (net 32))
 (segment (start 118.61 91.95) (end 117.46 93.1) (width 0.2) (layer "B.Cu") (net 32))
 (segment (start 167.46 93.1) (end 163.8898 93.1) (width 0.2) (layer "B.Cu") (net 32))
 (segment (start 163.8898 93.1) (end 162.7398 91.95) (width 0.2) (layer "B.Cu") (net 32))
 (segment (start 118.61 94.49) (end 117.46 95.64) (width 0.2) (layer "B.Cu") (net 34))
 (segment (start 162.689 94.49) (end 118.61 94.49) (width 0.2) (layer "B.Cu") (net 34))
 (segment (start 167.46 95.64) (end 163.839 95.64) (width 0.2) (layer "B.Cu") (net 34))
 (segment (start 163.839 95.64) (end 162.689 94.49) (width 0.2) (layer "B.Cu") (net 34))
 (segment (start 120 88.02) (end 162.4166 88.02) (width 0.2) (layer "B.Cu") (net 27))
 (segment (start 163.5666 89.17) (end 168.85 89.17) (width 0.2) (layer "B.Cu") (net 27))
 (segment (start 168.85 89.17) (end 170 88.02) (width 0.2) (layer "B.Cu") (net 27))
 (segment (start 162.4166 88.02) (end 163.5666 89.17) (width 0.2) (layer "B.Cu") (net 27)))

